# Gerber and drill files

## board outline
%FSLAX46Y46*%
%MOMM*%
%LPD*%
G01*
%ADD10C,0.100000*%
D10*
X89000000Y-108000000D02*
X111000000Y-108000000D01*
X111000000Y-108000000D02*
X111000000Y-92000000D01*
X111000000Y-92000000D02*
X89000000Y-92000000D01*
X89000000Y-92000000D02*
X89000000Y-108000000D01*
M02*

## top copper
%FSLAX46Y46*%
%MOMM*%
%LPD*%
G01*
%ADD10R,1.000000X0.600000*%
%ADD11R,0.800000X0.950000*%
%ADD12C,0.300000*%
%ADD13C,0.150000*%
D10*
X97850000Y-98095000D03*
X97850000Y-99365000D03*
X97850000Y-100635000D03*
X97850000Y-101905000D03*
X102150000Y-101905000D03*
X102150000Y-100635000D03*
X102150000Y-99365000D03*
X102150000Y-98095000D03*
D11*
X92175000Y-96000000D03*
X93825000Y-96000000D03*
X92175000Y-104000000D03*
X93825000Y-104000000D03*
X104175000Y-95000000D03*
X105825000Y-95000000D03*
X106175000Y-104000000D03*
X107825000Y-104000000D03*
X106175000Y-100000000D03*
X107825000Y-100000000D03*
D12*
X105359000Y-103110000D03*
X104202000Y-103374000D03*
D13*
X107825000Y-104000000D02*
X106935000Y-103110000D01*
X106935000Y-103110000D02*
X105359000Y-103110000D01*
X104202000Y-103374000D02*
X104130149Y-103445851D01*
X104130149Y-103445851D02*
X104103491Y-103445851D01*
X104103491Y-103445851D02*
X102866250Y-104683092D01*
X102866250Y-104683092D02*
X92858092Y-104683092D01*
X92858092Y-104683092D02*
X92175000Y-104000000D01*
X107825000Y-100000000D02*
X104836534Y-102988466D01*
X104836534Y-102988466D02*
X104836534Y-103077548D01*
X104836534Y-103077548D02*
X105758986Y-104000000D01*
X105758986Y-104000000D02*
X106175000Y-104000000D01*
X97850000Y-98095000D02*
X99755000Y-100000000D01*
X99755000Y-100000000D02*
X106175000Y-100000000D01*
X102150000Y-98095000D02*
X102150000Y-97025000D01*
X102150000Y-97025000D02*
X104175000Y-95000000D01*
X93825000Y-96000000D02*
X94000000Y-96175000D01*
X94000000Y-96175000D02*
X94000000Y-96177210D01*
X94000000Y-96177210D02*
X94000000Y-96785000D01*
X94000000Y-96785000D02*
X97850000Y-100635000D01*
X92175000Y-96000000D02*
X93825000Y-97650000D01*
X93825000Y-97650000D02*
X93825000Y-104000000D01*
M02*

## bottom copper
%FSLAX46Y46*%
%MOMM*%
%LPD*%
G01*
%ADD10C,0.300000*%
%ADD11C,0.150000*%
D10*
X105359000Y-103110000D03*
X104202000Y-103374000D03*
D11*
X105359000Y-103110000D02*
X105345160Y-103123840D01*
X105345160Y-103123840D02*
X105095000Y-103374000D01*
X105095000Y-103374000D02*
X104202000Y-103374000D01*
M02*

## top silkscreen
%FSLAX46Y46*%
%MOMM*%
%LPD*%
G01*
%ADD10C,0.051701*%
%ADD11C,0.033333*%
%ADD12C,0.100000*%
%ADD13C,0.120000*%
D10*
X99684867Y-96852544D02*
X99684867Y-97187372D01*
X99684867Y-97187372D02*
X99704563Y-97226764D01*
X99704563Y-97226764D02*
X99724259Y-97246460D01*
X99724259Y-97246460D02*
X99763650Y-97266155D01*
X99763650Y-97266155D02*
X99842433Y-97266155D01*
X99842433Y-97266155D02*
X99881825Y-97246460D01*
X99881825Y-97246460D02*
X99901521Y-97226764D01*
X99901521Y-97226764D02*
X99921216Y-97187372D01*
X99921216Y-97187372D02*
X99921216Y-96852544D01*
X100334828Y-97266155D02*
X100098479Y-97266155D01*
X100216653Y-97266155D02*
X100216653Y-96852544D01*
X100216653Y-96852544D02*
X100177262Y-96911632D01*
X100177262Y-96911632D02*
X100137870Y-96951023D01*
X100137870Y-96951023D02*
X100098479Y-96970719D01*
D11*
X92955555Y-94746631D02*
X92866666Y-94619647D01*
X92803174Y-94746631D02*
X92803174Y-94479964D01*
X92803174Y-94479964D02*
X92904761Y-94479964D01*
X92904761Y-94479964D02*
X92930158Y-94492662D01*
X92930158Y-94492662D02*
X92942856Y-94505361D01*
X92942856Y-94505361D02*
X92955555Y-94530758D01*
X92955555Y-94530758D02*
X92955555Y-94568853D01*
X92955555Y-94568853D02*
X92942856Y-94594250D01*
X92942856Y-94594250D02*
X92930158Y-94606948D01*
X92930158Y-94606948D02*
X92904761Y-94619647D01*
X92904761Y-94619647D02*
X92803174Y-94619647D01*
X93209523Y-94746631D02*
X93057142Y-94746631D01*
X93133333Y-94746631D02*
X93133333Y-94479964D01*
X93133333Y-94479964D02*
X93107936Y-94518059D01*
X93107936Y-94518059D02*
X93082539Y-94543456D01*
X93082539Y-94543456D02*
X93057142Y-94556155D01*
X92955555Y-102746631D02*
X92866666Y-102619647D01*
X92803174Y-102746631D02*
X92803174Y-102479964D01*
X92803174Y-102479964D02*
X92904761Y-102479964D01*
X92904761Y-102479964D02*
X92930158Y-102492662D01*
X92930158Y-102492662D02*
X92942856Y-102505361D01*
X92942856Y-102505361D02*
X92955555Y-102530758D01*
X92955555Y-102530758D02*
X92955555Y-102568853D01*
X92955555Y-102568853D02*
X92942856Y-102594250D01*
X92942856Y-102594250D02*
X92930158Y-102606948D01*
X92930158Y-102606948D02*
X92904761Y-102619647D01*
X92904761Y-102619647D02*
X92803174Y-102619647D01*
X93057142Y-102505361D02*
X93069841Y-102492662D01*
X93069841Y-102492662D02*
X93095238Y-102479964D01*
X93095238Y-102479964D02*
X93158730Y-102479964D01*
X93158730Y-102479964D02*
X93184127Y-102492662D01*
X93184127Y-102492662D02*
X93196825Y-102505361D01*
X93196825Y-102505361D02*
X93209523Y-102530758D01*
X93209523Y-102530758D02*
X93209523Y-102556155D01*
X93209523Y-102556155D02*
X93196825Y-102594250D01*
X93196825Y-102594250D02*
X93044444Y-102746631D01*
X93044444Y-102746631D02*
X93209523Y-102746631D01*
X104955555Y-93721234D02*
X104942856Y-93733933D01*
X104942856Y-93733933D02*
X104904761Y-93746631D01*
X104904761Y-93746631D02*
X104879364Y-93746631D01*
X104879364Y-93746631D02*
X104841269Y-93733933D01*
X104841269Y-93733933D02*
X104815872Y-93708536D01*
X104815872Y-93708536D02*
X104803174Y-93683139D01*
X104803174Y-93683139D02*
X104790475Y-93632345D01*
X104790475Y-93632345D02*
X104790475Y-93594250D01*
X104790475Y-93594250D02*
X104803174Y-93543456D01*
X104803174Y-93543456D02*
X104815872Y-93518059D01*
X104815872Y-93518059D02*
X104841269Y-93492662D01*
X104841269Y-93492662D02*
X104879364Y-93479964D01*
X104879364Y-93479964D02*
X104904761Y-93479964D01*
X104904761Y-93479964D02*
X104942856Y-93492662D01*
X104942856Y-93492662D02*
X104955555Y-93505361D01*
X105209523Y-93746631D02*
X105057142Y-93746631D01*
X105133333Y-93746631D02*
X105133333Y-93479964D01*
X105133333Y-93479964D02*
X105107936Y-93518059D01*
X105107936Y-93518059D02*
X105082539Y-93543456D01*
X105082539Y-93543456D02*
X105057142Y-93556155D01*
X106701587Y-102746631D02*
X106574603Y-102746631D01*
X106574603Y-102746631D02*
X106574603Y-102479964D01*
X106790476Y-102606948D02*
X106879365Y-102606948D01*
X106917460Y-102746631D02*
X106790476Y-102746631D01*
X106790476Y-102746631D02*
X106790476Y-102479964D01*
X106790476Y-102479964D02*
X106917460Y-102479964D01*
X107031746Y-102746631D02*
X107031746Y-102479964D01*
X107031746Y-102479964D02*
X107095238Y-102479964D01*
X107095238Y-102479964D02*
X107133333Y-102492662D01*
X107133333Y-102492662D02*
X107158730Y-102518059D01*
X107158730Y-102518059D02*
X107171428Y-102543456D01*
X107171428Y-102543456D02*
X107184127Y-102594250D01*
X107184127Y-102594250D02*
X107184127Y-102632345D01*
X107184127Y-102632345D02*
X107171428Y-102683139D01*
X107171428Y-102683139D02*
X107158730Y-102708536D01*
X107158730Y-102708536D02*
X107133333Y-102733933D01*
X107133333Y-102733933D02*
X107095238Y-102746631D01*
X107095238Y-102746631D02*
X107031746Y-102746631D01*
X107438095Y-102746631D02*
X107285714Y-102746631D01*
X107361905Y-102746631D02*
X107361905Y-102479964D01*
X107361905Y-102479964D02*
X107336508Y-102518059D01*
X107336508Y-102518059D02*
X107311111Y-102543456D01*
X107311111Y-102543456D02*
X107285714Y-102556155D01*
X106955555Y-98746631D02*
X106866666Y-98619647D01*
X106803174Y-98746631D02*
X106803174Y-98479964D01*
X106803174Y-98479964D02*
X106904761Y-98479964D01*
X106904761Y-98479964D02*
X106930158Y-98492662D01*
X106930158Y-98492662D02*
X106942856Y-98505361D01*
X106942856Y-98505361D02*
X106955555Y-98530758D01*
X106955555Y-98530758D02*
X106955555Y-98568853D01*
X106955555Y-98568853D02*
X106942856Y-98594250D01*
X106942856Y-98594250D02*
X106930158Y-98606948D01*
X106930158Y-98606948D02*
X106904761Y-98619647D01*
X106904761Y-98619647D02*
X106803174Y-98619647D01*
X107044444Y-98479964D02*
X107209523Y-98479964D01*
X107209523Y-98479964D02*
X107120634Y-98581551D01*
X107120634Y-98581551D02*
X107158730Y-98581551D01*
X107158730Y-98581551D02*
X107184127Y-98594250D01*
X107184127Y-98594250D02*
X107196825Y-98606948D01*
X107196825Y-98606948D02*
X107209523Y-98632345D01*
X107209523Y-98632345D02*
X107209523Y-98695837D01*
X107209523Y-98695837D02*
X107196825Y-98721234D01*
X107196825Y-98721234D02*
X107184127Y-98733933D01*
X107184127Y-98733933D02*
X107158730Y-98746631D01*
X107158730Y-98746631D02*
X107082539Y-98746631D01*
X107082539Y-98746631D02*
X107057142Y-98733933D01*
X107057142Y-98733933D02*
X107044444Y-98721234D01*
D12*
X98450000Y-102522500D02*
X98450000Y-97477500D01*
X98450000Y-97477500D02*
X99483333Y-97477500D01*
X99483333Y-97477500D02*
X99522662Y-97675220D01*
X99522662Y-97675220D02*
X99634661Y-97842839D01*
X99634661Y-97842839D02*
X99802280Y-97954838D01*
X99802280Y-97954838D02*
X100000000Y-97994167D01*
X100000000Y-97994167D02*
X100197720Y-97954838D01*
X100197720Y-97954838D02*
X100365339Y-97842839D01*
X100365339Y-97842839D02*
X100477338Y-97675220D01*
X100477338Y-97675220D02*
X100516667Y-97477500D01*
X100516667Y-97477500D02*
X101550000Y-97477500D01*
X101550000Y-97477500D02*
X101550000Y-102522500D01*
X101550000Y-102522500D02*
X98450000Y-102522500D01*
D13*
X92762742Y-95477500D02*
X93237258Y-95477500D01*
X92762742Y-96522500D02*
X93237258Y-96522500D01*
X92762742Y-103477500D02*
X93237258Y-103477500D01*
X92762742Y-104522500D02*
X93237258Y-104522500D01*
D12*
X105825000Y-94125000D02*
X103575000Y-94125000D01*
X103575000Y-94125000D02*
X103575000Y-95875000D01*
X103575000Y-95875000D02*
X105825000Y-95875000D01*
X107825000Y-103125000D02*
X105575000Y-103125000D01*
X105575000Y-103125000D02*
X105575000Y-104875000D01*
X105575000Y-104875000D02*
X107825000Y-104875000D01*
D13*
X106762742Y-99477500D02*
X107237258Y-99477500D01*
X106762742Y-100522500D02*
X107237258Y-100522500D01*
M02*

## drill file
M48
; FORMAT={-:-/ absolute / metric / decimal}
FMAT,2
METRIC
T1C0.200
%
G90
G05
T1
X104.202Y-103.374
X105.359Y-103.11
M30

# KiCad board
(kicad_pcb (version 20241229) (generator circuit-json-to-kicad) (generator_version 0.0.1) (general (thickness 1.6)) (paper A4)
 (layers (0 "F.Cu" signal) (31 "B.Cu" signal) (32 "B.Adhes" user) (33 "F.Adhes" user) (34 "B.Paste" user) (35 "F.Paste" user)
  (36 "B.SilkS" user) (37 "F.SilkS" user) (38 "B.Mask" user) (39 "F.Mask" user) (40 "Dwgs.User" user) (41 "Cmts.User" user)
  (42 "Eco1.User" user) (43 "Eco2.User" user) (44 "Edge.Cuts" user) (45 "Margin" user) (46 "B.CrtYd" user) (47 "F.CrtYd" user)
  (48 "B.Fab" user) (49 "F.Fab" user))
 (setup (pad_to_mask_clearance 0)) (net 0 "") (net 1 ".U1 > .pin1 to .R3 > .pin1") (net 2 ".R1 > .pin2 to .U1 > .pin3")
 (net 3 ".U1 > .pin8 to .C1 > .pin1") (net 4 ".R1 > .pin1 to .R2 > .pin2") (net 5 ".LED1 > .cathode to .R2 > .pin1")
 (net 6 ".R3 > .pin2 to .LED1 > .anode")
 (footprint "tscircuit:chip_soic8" (layer F.Cu) (at 100 100 0)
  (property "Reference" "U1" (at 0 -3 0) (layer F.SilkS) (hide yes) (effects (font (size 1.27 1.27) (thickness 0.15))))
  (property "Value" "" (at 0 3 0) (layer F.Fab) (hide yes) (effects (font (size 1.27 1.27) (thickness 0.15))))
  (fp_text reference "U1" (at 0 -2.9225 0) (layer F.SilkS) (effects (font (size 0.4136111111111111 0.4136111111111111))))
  (fp_line (start -1.5499999999999998 2.5225) (end -1.5499999999999998 -2.5225) (stroke (width 0.1) (type default)) (layer F.SilkS))
  (fp_line (start -1.5499999999999998 -2.5225) (end -0.5166666666666666 -2.5225) (stroke (width 0.1) (type default)) (layer F.SilkS))
  (fp_line (start -0.5166666666666666 -2.5225) (end -0.47733775846416476 -2.32478022661137) (stroke (width 0.1) (type default))
   (layer F.SilkS))
  (fp_line (start -0.47733775846416476 -2.32478022661137) (end -0.3653385036130495 -2.1571614963869505) (stroke (width 0.1) (type default))
   (layer F.SilkS))
  (fp_line (start -0.3653385036130495 -2.1571614963869505) (end -0.19771977338862967 -2.0451622415358353)
   (stroke (width 0.1) (type default)) (layer F.SilkS))
  (fp_line (start -0.19771977338862967 -2.0451622415358353) (end 3.1636708977973285e-17 -2.0058333333333334)
   (stroke (width 0.1) (type default)) (layer F.SilkS))
  (fp_line (start 3.1636708977973285e-17 -2.0058333333333334) (end 0.1977197733886297 -2.0451622415358353)
   (stroke (width 0.1) (type default)) (layer F.SilkS))
  (fp_line (start 0.1977197733886297 -2.0451622415358353) (end 0.3653385036130496 -2.1571614963869505) (stroke (width 0.1) (type default))
   (layer F.SilkS))
  (fp_line (start 0.3653385036130496 -2.1571614963869505) (end 0.47733775846416476 -2.32478022661137) (stroke (width 0.1) (type default))
   (layer F.SilkS))
  (fp_line (start 0.47733775846416476 -2.32478022661137) (end 0.5166666666666666 -2.5225) (stroke (width 0.1) (type default))
   (layer F.SilkS))
  (fp_line (start 0.5166666666666666 -2.5225) (end 1.5499999999999998 -2.5225) (stroke (width 0.1) (type default)) (layer F.SilkS))
  (fp_line (start 1.5499999999999998 -2.5225) (end 1.5499999999999998 2.5225) (stroke (width 0.1) (type default)) (layer F.SilkS))
  (fp_line (start 1.5499999999999998 2.5225) (end -1.5499999999999998 2.5225) (stroke (width 0.1) (type default)) (layer F.SilkS))
  (pad "1" smd rect (at -2.15 -1.905 0) (size 1 0.6) (layers F.Cu F.Paste F.Mask) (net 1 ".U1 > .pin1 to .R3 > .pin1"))
  (pad "2" smd rect (at -2.15 -0.635 0) (size 1 0.6) (layers F.Cu F.Paste F.Mask))
  (pad "3" smd rect (at -2.15 0.635 0) (size 1 0.6) (layers F.Cu F.Paste F.Mask) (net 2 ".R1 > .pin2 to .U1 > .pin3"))
  (pad "4" smd rect (at -2.15 1.905 0) (size 1 0.6) (layers F.Cu F.Paste F.Mask))
  (pad "5" smd rect (at 2.15 1.905 0) (size 1 0.6) (layers F.Cu F.Paste F.Mask))
  (pad "6" smd rect (at 2.15 0.635 0) (size 1 0.6) (layers F.Cu F.Paste F.Mask))
  (pad "7" smd rect (at 2.15 -0.635 0) (size 1 0.6) (layers F.Cu F.Paste F.Mask))
  (pad "8" smd rect (at 2.15 -1.905 0) (size 1 0.6) (layers F.Cu F.Paste F.Mask) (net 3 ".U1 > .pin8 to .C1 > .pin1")))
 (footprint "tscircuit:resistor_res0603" (layer F.Cu) (at 93 96 0)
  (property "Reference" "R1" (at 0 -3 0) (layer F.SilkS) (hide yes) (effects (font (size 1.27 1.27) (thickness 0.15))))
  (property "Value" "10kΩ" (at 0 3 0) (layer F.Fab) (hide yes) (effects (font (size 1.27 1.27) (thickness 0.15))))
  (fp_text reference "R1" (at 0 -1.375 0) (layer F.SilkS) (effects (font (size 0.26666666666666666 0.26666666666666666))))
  (fp_line (start -0.23725799999999975 -0.5225) (end 0.23725799999999975 -0.5225) (stroke (width 0.12) (type default)) (layer F.SilkS))
  (fp_line (start -0.23725799999999975 0.5225) (end 0.23725799999999975 0.5225) (stroke (width 0.12) (type default)) (layer F.SilkS))
  (pad "1" smd rect (at -0.8250000000000002 0 0) (size 0.8 0.95) (layers F.Cu F.Paste F.Mask) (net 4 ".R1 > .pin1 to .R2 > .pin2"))
  (pad "2" smd rect (at 0.8250000000000002 0 0) (size 0.8 0.95) (layers F.Cu F.Paste F.Mask) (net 2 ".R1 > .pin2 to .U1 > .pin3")))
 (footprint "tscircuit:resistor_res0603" (layer F.Cu) (at 93 104 0)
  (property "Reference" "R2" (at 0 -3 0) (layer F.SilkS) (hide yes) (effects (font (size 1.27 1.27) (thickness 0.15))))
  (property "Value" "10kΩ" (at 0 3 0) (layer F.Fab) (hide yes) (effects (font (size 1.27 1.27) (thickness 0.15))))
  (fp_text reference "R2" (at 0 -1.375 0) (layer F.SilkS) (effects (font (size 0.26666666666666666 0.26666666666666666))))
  (fp_line (start -0.23725799999999975 -0.5225) (end 0.23725799999999975 -0.5225) (stroke (width 0.12) (type default)) (layer F.SilkS))
  (fp_line (start -0.23725799999999975 0.5225) (end 0.23725799999999975 0.5225) (stroke (width 0.12) (type default)) (layer F.SilkS))
  (pad "1" smd rect (at -0.8250000000000002 0 0) (size 0.8 0.95) (layers F.Cu F.Paste F.Mask) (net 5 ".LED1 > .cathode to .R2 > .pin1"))
  (pad "2" smd rect (at 0.8250000000000002 0 0) (size 0.8 0.95) (layers F.Cu F.Paste F.Mask) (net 4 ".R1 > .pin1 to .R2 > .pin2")))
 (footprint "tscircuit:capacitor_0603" (layer F.Cu) (at 105 95 0)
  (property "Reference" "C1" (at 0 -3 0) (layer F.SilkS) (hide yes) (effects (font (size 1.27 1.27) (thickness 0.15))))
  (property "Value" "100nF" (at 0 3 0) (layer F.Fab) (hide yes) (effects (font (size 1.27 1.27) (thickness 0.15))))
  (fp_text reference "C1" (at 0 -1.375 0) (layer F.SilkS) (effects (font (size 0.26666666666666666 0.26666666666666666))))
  (fp_line (start 0.8250000000000002 -0.875) (end -1.4249999999999998 -0.875) (stroke (width 0.1) (type default)) (layer F.SilkS))
  (fp_line (start -1.4249999999999998 -0.875) (end -1.4249999999999998 0.875) (stroke (width 0.1) (type default)) (layer F.SilkS))
  (fp_line (start -1.4249999999999998 0.875) (end 0.8250000000000002 0.875) (stroke (width 0.1) (type default)) (layer F.SilkS))
  (pad "1" smd rect (at -0.8250000000000002 0 0) (size 0.8 0.95) (layers F.Cu F.Paste F.Mask) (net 3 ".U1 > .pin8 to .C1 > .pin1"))
  (pad "2" smd rect (at 0.8250000000000002 0 0) (size 0.8 0.95) (layers F.Cu F.Paste F.Mask)))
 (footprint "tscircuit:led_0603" (layer F.Cu) (at 107 104 0)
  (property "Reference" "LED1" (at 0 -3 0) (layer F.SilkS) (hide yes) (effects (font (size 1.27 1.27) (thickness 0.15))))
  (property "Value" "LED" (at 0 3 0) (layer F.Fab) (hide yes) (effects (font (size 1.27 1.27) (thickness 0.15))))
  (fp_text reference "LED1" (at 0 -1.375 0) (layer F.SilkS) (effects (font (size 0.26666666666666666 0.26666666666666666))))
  (fp_line (start 0.8250000000000002 -0.875) (end -1.4249999999999998 -0.875) (stroke (width 0.1) (type default)) (layer F.SilkS))
  (fp_line (start -1.4249999999999998 -0.875) (end -1.4249999999999998 0.875) (stroke (width 0.1) (type default)) (layer F.SilkS))
  (fp_line (start -1.4249999999999998 0.875) (end 0.8250000000000002 0.875) (stroke (width 0.1) (type default)) (layer F.SilkS))
  (pad "1" smd rect (at -0.8250000000000002 0 0) (size 0.8 0.95) (layers F.Cu F.Paste F.Mask) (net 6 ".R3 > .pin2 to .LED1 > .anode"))
  (pad "2" smd rect (at 0.8250000000000002 0 0) (size 0.8 0.95) (layers F.Cu F.Paste F.Mask) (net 5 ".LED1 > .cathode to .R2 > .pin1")))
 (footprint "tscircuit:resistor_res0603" (layer F.Cu) (at 107 100 0)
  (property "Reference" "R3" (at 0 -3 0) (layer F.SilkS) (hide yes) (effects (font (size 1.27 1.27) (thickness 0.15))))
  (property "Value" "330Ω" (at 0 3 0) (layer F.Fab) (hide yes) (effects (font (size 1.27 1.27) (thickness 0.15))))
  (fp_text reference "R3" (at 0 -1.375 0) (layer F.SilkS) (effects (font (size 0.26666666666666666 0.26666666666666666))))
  (fp_line (start -0.23725799999999975 -0.5225) (end 0.23725799999999975 -0.5225) (stroke (width 0.12) (type default)) (layer F.SilkS))
  (fp_line (start -0.23725799999999975 0.5225) (end 0.23725799999999975 0.5225) (stroke (width 0.12) (type default)) (layer F.SilkS))
  (pad "1" smd rect (at -0.8250000000000002 0 0) (size 0.8 0.95) (layers F.Cu F.Paste F.Mask) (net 1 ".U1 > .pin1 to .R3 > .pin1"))
  (pad "2" smd rect (at 0.8250000000000002 0 0) (size 0.8 0.95) (layers F.Cu F.Paste F.Mask) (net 6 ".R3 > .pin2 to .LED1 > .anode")))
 (segment (start 107.825 104) (end 106.935 103.11) (width 0.15) (layer F.Cu) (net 5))
 (segment (start 106.935 103.11) (end 105.359 103.11) (width 0.15) (layer F.Cu) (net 5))
 (segment (start 105.359 103.11) (end 105.34515950363469 103.1238404963653) (width 0.15) (layer B.Cu) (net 5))
 (segment (start 105.34515950363469 103.1238404963653) (end 105.095 103.374) (width 0.15) (layer B.Cu) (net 5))
 (segment (start 105.095 103.374) (end 104.202 103.374) (width 0.15) (layer B.Cu) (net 5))
 (segment (start 104.202 103.374) (end 104.13014900286876 103.44585099713125) (width 0.15) (layer F.Cu) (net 5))
 (segment (start 104.13014900286876 103.44585099713125) (end 104.10349085714178 103.44585099713125) (width 0.15) (layer F.Cu) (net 5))
 (segment (start 104.10349085714178 103.44585099713125) (end 102.86625020159133 104.6830916526817) (width 0.15) (layer F.Cu) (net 5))
 (segment (start 102.86625020159133 104.6830916526817) (end 92.8580916526817 104.6830916526817) (width 0.15) (layer F.Cu) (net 5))
 (segment (start 92.8580916526817 104.6830916526817) (end 92.175 104) (width 0.15) (layer F.Cu) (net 5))
 (segment (start 107.825 100) (end 104.83653412921323 102.98846587078677) (width 0.15) (layer F.Cu) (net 6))
 (segment (start 104.83653412921323 102.98846587078677) (end 104.83653412921323 103.07754812385483) (width 0.15) (layer F.Cu) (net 6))
 (segment (start 104.83653412921323 103.07754812385483) (end 105.7589860053584 104) (width 0.15) (layer F.Cu) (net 6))
 (segment (start 105.7589860053584 104) (end 106.175 104) (width 0.15) (layer F.Cu) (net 6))
 (segment (start 97.85 98.095) (end 99.755 100) (width 0.15) (layer F.Cu) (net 1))
 (segment (start 99.755 100) (end 106.175 100) (width 0.15) (layer F.Cu) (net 1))
 (segment (start 102.15 98.095) (end 102.15 97.025) (width 0.15) (layer F.Cu) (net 3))
 (segment (start 102.15 97.025) (end 104.175 95) (width 0.15) (layer F.Cu) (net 3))
 (segment (start 93.825 96) (end 94 96.175) (width 0.15) (layer F.Cu) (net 2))
 (segment (start 94 96.175) (end 94 96.1772096342315) (width 0.15) (layer F.Cu) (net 2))
 (segment (start 94 96.1772096342315) (end 94 96.785) (width 0.15) (layer F.Cu) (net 2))
 (segment (start 94 96.785) (end 97.85 100.635) (width 0.15) (layer F.Cu) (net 2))
 (segment (start 92.175 96) (end 93.825 97.65) (width 0.15) (layer F.Cu) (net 4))
 (segment (start 93.825 97.65) (end 93.825 104) (width 0.15) (layer F.Cu) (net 4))
 (gr_line (start 89 108) (end 111 108) (width 0.1) (layer Edge.Cuts))
 (gr_line (start 111 108) (end 111 92) (width 0.1) (layer Edge.Cuts))
 (gr_line (start 111 92) (end 89 92) (width 0.1) (layer Edge.Cuts))
 (gr_line (start 89 92) (end 89 108) (width 0.1) (layer Edge.Cuts))
 (via (at 105.359 103.11) (size 0.3) (drill 0.2) (layers F.Cu B.Cu) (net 5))
 (via (at 104.202 103.374) (size 0.3) (drill 0.2) (layers F.Cu B.Cu) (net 5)))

